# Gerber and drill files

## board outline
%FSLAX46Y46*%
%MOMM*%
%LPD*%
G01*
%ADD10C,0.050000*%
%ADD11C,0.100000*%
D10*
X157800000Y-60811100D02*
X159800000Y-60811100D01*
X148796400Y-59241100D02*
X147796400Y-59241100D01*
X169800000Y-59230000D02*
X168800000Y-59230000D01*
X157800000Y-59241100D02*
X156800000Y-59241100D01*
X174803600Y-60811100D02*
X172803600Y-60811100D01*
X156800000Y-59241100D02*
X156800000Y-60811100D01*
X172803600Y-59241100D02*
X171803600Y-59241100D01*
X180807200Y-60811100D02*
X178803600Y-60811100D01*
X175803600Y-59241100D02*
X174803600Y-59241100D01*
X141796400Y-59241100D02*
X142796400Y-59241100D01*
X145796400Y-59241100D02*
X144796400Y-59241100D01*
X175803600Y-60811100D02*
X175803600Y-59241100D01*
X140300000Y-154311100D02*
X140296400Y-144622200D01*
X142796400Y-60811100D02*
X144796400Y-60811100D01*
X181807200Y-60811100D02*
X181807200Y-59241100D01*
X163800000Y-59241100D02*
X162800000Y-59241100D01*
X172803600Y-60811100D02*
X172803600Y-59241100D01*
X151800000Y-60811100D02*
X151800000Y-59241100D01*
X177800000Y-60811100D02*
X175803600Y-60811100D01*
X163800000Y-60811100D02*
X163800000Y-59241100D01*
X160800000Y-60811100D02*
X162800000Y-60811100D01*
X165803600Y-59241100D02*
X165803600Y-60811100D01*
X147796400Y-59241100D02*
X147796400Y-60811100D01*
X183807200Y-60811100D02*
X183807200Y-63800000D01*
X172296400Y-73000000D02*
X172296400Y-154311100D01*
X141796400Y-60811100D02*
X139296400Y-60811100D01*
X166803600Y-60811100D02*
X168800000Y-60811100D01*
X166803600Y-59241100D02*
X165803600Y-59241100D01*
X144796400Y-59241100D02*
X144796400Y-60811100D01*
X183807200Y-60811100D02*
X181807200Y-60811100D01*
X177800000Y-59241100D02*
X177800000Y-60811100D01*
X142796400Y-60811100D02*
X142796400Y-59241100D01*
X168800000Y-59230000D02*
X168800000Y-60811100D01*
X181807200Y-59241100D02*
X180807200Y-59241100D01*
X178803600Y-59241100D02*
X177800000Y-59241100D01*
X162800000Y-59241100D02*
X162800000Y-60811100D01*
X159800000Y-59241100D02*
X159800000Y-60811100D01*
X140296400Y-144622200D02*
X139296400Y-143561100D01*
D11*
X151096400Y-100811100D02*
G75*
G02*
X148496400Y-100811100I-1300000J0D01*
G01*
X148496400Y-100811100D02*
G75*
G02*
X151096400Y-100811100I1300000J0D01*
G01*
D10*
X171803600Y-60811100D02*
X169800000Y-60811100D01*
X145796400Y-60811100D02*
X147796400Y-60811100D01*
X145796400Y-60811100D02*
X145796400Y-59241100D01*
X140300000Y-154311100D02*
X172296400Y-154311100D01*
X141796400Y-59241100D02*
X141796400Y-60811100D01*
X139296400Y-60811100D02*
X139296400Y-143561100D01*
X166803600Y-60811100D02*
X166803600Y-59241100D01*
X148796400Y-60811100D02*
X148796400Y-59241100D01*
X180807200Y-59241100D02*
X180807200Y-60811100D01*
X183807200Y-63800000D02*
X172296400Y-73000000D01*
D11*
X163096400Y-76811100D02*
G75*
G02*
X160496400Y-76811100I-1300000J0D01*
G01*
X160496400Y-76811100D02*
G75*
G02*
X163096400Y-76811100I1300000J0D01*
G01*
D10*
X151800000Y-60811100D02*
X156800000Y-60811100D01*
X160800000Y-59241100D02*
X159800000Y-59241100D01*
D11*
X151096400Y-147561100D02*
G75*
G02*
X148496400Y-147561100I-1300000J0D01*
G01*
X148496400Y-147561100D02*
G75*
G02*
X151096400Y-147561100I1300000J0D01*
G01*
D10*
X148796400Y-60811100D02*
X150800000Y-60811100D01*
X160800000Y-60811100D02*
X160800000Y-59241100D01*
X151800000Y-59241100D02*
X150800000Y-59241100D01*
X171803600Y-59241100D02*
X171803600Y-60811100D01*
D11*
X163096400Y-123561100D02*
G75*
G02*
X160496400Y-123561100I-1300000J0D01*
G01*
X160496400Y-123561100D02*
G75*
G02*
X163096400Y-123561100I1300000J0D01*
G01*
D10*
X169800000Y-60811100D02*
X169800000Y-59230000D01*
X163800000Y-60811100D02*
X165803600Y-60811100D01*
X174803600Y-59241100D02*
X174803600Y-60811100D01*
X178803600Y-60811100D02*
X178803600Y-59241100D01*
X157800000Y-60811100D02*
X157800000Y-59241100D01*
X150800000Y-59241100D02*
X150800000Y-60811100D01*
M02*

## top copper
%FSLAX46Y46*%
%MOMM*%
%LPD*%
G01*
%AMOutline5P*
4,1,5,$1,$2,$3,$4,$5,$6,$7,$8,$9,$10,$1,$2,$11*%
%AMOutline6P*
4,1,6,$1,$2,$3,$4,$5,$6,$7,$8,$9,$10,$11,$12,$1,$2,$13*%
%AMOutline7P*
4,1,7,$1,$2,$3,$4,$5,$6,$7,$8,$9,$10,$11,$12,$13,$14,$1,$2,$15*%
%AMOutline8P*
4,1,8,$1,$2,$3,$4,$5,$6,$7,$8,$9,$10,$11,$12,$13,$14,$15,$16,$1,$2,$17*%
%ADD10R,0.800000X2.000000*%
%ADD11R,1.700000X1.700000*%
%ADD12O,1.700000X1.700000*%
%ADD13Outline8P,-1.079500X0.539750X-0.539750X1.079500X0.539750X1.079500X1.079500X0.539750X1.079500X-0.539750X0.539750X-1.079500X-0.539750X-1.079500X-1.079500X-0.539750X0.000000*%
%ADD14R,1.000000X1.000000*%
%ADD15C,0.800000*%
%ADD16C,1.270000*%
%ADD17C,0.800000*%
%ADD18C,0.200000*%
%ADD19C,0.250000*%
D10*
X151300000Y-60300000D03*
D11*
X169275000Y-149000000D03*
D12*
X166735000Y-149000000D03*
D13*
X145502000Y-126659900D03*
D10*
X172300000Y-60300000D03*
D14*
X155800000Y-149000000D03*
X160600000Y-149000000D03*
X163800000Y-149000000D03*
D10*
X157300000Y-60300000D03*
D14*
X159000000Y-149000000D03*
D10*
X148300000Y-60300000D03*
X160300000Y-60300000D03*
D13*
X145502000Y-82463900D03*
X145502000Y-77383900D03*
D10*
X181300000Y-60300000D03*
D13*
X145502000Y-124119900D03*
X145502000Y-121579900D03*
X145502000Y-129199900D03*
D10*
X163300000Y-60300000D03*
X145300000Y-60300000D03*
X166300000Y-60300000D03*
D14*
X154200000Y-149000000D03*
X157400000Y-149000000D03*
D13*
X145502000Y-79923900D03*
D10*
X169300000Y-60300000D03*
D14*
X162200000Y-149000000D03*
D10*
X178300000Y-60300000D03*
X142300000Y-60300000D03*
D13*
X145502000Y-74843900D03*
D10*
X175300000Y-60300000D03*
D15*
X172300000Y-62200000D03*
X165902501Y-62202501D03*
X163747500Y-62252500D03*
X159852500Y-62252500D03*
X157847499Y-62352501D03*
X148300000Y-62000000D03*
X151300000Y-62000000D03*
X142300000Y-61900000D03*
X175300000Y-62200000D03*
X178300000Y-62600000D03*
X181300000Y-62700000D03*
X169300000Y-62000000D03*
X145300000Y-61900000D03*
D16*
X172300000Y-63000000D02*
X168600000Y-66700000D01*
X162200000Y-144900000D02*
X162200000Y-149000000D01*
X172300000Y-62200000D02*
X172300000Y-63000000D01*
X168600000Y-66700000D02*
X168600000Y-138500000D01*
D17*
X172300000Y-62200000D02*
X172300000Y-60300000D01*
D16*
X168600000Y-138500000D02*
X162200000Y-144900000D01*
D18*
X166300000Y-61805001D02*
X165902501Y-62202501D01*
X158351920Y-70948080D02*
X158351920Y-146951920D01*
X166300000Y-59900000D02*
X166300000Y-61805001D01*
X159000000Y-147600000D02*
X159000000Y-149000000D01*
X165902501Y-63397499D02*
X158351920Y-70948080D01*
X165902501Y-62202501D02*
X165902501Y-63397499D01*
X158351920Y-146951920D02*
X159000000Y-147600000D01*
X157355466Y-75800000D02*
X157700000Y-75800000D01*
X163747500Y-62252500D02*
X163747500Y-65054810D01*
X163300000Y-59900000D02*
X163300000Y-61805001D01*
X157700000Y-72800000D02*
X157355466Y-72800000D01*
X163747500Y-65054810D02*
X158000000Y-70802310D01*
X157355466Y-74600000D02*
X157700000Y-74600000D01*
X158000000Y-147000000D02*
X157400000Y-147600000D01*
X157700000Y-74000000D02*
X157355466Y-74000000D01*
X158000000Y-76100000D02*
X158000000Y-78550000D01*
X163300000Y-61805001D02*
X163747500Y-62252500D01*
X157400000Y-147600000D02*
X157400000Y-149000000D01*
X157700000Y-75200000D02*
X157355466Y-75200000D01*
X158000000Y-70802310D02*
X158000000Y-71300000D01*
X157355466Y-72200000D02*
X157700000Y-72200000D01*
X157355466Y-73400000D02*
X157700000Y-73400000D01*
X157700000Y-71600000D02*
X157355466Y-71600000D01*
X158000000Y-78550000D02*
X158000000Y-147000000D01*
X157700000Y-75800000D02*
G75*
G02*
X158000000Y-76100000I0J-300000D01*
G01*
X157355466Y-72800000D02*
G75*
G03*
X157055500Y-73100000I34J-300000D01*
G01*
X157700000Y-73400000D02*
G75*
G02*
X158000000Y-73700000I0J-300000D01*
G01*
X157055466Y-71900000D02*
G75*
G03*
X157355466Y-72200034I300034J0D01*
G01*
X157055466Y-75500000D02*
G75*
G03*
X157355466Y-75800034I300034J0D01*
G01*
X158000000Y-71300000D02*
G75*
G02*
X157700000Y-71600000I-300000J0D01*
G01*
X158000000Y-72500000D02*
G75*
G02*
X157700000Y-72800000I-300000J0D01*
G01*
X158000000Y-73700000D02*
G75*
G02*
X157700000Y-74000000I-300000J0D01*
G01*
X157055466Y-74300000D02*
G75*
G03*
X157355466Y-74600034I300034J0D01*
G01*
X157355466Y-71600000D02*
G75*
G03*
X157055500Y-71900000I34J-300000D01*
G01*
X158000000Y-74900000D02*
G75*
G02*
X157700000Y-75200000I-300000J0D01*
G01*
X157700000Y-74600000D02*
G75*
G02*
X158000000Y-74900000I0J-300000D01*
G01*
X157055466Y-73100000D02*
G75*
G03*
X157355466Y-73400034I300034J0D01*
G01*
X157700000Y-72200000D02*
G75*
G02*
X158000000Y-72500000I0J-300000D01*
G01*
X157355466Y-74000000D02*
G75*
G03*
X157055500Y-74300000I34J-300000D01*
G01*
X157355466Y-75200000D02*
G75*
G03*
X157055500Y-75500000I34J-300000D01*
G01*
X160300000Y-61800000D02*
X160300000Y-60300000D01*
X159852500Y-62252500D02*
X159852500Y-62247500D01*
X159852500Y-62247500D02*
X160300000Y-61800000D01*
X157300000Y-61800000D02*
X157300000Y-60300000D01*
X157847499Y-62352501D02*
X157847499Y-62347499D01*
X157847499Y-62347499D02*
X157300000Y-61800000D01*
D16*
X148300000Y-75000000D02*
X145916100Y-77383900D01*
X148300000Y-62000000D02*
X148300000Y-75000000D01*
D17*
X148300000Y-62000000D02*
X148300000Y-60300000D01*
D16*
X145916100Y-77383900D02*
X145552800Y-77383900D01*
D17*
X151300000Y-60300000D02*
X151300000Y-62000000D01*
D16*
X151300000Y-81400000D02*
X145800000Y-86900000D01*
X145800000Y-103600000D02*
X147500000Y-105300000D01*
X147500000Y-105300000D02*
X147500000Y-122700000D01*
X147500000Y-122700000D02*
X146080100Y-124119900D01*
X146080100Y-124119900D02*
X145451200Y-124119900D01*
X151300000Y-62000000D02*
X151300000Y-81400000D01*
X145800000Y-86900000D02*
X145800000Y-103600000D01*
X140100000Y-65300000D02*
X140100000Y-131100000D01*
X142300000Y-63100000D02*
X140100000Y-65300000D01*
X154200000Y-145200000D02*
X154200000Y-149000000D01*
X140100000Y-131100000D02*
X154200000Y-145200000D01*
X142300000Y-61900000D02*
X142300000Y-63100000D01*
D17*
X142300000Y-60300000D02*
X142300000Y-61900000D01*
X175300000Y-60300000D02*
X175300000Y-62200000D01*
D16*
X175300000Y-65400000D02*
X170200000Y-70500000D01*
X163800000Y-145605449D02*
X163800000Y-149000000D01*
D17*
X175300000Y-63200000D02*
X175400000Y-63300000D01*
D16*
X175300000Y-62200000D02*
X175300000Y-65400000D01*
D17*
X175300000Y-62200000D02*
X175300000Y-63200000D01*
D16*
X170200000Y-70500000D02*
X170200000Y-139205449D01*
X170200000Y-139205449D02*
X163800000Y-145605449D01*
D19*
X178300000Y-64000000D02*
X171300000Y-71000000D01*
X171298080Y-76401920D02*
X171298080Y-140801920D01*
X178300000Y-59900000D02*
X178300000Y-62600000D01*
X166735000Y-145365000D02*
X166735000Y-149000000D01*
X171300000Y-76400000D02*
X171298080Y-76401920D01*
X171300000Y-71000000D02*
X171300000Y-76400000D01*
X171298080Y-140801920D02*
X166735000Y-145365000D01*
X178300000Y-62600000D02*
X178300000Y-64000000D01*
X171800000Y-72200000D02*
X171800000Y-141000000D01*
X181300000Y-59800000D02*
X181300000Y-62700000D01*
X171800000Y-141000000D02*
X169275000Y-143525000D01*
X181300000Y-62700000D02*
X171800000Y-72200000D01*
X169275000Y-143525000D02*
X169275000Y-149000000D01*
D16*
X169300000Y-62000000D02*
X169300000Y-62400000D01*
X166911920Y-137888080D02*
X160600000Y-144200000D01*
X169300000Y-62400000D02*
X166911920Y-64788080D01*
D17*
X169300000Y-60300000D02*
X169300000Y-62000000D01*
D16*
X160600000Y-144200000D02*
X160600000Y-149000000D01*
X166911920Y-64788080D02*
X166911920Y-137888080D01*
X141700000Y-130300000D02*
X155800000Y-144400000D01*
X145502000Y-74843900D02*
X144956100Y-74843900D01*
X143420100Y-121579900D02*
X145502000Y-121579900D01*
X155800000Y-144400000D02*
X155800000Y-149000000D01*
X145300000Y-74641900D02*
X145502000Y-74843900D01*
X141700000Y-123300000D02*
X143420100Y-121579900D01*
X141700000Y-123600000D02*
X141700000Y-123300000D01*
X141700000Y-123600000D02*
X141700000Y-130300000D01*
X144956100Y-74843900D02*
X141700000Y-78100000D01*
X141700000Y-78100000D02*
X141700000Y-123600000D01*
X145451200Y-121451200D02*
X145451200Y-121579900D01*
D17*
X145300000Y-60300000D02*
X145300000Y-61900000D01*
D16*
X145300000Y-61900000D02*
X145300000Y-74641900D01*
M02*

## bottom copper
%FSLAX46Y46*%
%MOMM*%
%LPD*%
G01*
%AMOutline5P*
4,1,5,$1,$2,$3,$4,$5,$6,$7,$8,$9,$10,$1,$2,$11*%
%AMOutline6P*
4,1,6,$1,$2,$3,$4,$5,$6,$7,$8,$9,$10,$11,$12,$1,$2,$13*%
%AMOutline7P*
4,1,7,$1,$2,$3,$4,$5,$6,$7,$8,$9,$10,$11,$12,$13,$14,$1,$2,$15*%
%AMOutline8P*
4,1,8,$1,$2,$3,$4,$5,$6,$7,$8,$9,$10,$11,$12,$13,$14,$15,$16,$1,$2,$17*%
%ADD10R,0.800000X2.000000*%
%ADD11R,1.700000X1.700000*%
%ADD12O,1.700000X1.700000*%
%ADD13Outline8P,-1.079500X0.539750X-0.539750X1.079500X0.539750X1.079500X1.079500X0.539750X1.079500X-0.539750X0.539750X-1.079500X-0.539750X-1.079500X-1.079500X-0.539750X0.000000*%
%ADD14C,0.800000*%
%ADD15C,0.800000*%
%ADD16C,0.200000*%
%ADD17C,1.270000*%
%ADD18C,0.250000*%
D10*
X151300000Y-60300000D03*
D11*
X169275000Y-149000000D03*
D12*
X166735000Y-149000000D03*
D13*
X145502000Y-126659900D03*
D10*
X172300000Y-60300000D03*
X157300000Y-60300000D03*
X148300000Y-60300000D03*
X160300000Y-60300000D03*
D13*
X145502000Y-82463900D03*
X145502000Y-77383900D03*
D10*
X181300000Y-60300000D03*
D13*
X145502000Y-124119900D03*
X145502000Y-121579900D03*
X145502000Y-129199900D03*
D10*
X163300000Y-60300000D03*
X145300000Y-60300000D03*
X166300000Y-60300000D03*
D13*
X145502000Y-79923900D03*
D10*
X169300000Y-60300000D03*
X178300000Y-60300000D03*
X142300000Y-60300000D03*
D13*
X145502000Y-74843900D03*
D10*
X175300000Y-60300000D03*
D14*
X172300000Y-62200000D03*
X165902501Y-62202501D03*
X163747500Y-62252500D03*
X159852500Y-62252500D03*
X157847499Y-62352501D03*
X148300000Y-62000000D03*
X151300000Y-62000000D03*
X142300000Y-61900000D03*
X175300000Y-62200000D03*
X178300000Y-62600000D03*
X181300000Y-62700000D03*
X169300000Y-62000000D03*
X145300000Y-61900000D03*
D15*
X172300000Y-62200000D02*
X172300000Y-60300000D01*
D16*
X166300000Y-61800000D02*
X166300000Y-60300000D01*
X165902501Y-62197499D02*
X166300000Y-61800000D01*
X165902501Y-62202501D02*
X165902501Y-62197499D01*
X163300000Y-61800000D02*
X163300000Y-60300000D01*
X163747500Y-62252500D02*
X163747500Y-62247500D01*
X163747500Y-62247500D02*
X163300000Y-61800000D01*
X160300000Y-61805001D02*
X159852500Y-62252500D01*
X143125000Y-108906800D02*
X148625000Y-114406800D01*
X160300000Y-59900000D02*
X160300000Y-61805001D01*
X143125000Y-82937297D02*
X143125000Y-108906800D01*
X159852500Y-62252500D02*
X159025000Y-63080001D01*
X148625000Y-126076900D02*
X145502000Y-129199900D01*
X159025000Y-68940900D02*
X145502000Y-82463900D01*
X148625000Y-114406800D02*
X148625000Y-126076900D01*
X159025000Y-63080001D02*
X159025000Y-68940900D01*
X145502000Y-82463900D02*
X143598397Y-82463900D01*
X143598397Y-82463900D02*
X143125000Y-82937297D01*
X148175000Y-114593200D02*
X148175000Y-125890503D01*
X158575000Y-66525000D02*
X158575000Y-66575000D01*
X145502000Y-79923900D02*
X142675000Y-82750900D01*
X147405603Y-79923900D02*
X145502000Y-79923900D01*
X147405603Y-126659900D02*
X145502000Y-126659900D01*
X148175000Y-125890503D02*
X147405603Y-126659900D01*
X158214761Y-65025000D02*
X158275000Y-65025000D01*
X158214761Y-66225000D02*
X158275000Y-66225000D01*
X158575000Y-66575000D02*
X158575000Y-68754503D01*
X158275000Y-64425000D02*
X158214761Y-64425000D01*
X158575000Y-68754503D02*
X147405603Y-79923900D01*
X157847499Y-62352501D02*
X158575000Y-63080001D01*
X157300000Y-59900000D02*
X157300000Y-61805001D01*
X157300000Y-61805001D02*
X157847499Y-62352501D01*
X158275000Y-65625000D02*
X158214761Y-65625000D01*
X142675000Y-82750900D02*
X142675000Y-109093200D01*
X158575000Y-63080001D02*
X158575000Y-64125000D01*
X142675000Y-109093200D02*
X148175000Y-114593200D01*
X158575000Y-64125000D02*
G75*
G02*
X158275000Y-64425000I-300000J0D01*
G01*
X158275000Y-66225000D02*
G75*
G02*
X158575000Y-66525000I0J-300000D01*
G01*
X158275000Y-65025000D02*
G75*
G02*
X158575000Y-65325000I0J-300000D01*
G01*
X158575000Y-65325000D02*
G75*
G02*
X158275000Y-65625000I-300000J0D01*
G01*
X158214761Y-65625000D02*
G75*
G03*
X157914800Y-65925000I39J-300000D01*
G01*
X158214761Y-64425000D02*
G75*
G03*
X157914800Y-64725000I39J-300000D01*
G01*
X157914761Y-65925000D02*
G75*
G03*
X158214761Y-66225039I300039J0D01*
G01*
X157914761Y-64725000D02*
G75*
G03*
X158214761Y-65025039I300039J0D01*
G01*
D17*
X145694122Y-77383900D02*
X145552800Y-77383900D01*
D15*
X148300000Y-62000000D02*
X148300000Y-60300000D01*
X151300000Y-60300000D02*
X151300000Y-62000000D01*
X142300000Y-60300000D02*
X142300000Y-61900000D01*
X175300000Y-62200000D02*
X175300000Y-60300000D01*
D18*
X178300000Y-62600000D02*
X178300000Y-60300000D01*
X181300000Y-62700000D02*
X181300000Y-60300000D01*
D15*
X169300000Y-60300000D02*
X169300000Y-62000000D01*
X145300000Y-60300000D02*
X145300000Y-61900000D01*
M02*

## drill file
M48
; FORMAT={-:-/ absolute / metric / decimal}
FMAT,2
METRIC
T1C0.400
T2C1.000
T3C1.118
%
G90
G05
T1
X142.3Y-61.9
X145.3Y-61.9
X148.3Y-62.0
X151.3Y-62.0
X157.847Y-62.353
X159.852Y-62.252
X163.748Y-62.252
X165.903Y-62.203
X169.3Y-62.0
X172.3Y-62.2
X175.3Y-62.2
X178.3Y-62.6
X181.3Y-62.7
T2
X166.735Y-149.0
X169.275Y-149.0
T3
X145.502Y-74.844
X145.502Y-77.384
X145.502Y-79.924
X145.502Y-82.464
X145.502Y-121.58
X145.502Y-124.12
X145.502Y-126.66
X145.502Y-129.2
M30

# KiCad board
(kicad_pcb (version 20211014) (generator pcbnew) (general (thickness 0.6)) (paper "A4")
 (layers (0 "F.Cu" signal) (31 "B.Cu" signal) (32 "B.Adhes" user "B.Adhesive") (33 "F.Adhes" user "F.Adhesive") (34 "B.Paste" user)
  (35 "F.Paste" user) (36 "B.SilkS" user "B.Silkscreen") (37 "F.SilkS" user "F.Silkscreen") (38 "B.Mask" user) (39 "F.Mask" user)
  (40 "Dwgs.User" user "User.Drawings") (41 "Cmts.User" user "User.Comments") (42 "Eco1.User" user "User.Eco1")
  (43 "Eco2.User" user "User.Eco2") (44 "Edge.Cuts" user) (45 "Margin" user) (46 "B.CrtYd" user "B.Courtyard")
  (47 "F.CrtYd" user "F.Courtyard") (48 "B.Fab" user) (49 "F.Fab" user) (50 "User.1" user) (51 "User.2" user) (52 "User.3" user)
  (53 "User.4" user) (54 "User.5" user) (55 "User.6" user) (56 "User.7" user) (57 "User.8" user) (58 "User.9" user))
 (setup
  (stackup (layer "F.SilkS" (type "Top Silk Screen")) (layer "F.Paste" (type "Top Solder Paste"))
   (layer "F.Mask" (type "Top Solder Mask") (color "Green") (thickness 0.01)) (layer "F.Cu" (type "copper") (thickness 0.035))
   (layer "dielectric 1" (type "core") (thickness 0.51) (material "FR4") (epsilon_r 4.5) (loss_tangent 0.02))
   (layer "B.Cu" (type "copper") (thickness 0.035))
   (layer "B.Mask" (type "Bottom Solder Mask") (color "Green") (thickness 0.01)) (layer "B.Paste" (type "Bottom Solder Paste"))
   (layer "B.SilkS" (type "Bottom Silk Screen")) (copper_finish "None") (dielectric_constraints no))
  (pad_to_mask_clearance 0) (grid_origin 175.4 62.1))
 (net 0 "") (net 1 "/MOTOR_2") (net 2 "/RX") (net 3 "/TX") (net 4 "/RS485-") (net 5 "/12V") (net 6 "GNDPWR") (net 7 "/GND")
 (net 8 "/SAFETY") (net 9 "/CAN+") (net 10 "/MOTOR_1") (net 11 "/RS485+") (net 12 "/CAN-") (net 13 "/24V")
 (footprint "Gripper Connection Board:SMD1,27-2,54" (layer "F.Cu") (at 151.3 60.3)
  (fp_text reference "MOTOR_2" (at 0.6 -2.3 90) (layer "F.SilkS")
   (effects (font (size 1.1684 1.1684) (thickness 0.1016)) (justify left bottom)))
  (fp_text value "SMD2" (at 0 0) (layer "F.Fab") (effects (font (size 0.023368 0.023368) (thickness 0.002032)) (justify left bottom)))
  (pad "1" smd rect (at 0 0) (size 0.8 2) (layers "F.Cu" "F.Paste" "F.Mask") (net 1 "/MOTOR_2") (solder_mask_margin 0.1016))
  (pad "2" smd rect (at 0 0) (size 0.8 2) (layers "B.Cu" "B.Paste" "B.Mask") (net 1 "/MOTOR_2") (solder_mask_margin 0.1016)))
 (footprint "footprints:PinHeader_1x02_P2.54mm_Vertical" (layer "F.Cu") (at 169.275 149 -90)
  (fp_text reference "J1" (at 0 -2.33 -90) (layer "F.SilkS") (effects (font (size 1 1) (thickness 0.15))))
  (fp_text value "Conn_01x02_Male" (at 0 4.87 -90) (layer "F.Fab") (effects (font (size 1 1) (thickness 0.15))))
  (pad "1" thru_hole rect locked (at 0 0 270) (size 1.7 1.7) (drill 1) (layers *.Cu *.Mask) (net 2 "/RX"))
  (pad "2" thru_hole oval locked (at 0 2.54 270) (size 1.7 1.7) (drill 1) (layers *.Cu *.Mask) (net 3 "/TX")))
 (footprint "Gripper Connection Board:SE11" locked (layer "F.Cu") (at 145.502 126.6599)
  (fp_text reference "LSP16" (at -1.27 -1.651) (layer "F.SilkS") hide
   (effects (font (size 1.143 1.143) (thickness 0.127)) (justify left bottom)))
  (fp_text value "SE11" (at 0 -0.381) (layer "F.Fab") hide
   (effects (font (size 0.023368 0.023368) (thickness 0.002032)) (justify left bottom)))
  (pad "MP" thru_hole roundrect locked (at 0 0) (size 2.159 2.159) (drill 1.1176) (layers *.Cu *.Mask) (roundrect_rratio 0.25)
   (chamfer_ratio 0.25) (chamfer top_left top_right bottom_left bottom_right) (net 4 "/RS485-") (solder_mask_margin 0.1016)))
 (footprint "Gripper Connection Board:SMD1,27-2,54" (layer "F.Cu") (at 172.3 60.3)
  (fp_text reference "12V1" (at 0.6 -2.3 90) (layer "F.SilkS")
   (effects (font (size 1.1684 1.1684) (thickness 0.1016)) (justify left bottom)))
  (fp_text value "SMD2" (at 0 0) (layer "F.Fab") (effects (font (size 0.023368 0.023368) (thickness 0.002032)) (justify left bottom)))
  (pad "1" smd rect (at 0 0) (size 0.8 2) (layers "F.Cu" "F.Paste" "F.Mask") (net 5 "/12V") (solder_mask_margin 0.1016))
  (pad "2" smd rect (at 0 0) (size 0.8 2) (layers "B.Cu" "B.Paste" "B.Mask") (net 5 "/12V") (solder_mask_margin 0.1016)))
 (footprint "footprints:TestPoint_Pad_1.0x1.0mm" (layer "F.Cu") (at 155.8 149)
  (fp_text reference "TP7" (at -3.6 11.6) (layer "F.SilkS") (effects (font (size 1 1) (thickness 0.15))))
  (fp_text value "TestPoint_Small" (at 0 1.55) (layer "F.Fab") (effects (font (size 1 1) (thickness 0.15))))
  (pad "1" smd rect locked (at 0 0) (size 1 1) (layers "F.Cu" "F.Mask") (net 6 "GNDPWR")))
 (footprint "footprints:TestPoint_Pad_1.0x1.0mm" (layer "F.Cu") (at 160.6 149)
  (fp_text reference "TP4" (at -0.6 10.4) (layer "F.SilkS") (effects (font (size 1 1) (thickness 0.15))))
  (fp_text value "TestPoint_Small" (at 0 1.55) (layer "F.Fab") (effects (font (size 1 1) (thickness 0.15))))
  (pad "1" smd rect locked (at 0 0) (size 1 1) (layers "F.Cu" "F.Mask") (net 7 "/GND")))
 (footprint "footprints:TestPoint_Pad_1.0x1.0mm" (layer "F.Cu") (at 163.8 149)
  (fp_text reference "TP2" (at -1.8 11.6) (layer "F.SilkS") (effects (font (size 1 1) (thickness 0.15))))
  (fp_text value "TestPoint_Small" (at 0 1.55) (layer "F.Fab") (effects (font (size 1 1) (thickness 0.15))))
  (pad "1" smd rect locked (at 0 0) (size 1 1) (layers "F.Cu" "F.Mask") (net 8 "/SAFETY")))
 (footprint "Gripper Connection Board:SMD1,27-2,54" (layer "F.Cu") (at 157.3 60.3)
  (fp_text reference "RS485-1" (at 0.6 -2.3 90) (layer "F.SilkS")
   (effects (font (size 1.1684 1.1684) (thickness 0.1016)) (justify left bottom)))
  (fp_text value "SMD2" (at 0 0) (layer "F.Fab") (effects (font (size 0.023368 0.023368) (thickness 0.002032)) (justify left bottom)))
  (pad "1" smd rect (at 0 0) (size 0.8 2) (layers "F.Cu" "F.Paste" "F.Mask") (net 4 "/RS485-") (solder_mask_margin 0.1016))
  (pad "2" smd rect (at 0 0) (size 0.8 2) (layers "B.Cu" "B.Paste" "B.Mask") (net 4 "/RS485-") (solder_mask_margin 0.1016)))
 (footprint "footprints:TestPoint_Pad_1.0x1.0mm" (layer "F.Cu") (at 159 149)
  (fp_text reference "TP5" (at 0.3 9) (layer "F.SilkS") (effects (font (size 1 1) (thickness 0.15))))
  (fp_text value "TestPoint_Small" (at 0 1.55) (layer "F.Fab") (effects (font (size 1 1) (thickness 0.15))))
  (pad "1" smd rect locked (at 0 0) (size 1 1) (layers "F.Cu" "F.Mask") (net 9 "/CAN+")))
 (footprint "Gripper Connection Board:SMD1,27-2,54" (layer "F.Cu") (at 148.3 60.3)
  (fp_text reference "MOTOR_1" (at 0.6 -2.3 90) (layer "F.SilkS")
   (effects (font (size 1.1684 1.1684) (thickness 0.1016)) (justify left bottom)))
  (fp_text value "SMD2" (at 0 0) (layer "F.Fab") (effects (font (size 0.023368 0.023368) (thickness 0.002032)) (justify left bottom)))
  (pad "1" smd rect (at 0 0) (size 0.8 2) (layers "F.Cu" "F.Paste" "F.Mask") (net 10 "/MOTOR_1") (solder_mask_margin 0.1016))
  (pad "2" smd rect (at 0 0) (size 0.8 2) (layers "B.Cu" "B.Paste" "B.Mask") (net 10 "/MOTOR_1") (solder_mask_margin 0.1016)))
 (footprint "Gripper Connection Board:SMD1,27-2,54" (layer "F.Cu") (at 160.3 60.3)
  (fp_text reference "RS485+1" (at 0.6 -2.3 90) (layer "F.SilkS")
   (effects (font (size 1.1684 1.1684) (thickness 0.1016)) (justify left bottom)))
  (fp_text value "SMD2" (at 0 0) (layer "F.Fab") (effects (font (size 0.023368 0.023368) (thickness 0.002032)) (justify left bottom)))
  (pad "1" smd rect (at 0 0) (size 0.8 2) (layers "F.Cu" "F.Paste" "F.Mask") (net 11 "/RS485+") (solder_mask_margin 0.1016))
  (pad "2" smd rect (at 0 0) (size 0.8 2) (layers "B.Cu" "B.Paste" "B.Mask") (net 11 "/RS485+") (solder_mask_margin 0.1016)))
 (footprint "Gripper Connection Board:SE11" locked (layer "F.Cu") (at 145.502 82.4639)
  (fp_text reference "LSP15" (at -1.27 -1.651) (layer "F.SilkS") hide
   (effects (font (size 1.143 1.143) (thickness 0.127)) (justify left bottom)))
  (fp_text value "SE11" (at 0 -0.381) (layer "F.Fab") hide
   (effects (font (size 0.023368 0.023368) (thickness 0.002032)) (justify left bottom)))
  (pad "MP" thru_hole roundrect locked (at 0 0) (size 2.159 2.159) (drill 1.1176) (layers *.Cu *.Mask) (roundrect_rratio 0.25)
   (chamfer_ratio 0.25) (chamfer top_left top_right bottom_left bottom_right) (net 11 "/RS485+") (solder_mask_margin 0.1016)))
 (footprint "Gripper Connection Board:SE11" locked (layer "F.Cu") (at 145.502 77.3839)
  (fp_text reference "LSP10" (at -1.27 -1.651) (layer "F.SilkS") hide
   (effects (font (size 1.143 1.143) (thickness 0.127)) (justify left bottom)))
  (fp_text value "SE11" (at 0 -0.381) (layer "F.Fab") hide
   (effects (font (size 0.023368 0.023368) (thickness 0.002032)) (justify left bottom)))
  (pad "MP" thru_hole roundrect locked (at 0 0) (size 2.159 2.159) (drill 1.1176) (layers *.Cu *.Mask) (roundrect_rratio 0.25)
   (chamfer_ratio 0.25) (chamfer top_left top_right bottom_left bottom_right) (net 10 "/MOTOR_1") (solder_mask_margin 0.1016)))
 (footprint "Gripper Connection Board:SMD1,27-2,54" (layer "F.Cu") (at 181.3 60.3)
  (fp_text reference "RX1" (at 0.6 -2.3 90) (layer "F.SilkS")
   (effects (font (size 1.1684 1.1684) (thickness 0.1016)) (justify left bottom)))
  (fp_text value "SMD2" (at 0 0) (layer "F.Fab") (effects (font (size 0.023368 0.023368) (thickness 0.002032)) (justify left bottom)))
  (pad "1" smd rect (at 0 0) (size 0.8 2) (layers "F.Cu" "F.Paste" "F.Mask") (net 2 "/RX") (solder_mask_margin 0.1016))
  (pad "2" smd rect (at 0 0) (size 0.8 2) (layers "B.Cu" "B.Paste" "B.Mask") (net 2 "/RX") (solder_mask_margin 0.1016)))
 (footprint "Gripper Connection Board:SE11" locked (layer "F.Cu") (at 145.502 124.1199)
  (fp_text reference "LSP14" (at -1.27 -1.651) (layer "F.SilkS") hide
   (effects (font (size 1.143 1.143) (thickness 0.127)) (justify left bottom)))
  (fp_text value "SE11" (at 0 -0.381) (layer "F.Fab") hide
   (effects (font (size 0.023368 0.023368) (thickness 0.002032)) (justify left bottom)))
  (pad "MP" thru_hole roundrect locked (at 0 0) (size 2.159 2.159) (drill 1.1176) (layers *.Cu *.Mask) (roundrect_rratio 0.25)
   (chamfer_ratio 0.25) (chamfer top_left top_right bottom_left bottom_right) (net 1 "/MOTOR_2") (solder_mask_margin 0.1016)))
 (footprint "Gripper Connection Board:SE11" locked (layer "F.Cu") (at 145.502 121.5799)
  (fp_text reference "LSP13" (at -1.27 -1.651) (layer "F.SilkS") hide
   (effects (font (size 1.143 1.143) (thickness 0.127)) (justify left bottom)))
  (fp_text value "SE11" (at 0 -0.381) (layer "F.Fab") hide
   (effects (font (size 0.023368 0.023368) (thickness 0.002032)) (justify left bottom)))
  (pad "MP" thru_hole roundrect locked (at 0 0) (size 2.159 2.159) (drill 1.1176) (layers *.Cu *.Mask) (roundrect_rratio 0.25)
   (chamfer_ratio 0.25) (chamfer top_left top_right bottom_left bottom_right) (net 6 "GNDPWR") (solder_mask_margin 0.1016)))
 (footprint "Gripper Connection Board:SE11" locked (layer "F.Cu") (at 145.502 129.1999)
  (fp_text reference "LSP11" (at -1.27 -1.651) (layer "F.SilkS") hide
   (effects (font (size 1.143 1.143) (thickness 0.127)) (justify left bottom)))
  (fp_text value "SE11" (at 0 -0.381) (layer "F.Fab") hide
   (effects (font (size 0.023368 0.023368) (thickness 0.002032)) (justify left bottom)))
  (pad "MP" thru_hole roundrect locked (at 0 0) (size 2.159 2.159) (drill 1.1176) (layers *.Cu *.Mask) (roundrect_rratio 0.25)
   (chamfer_ratio 0.25) (chamfer top_left top_right bottom_left bottom_right) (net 11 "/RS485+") (solder_mask_margin 0.1016)))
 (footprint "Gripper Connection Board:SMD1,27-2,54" (layer "F.Cu") (at 163.3 60.3)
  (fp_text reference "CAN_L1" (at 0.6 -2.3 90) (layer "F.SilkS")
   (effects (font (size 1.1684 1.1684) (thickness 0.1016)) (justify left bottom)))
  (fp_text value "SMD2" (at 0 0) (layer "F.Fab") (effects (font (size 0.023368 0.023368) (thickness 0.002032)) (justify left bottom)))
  (pad "1" smd rect (at 0 0) (size 0.8 2) (layers "F.Cu" "F.Paste" "F.Mask") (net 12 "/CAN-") (solder_mask_margin 0.1016))
  (pad "2" smd rect (at 0 0) (size 0.8 2) (layers "B.Cu" "B.Paste" "B.Mask") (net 12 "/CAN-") (solder_mask_margin 0.1016)))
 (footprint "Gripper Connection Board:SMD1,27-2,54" (layer "F.Cu") (at 145.3 60.3)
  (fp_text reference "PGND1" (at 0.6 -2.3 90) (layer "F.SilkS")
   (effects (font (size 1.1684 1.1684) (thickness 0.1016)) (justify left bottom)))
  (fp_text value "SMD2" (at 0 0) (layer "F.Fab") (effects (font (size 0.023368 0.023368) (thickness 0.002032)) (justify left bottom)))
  (pad "1" smd rect (at 0 0) (size 0.8 2) (layers "F.Cu" "F.Paste" "F.Mask") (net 6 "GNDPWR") (solder_mask_margin 0.1016))
  (pad "2" smd rect (at 0 0) (size 0.8 2) (layers "B.Cu" "B.Paste" "B.Mask") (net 6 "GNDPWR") (solder_mask_margin 0.1016)))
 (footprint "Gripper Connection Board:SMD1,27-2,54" (layer "F.Cu") (at 166.3 60.3)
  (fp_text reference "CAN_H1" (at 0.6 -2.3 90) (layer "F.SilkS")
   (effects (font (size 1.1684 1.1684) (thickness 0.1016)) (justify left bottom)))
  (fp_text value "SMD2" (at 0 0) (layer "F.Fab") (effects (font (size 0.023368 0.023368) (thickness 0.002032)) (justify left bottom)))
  (pad "1" smd rect (at 0 0) (size 0.8 2) (layers "F.Cu" "F.Paste" "F.Mask") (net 9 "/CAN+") (solder_mask_margin 0.1016))
  (pad "2" smd rect (at 0 0) (size 0.8 2) (layers "B.Cu" "B.Paste" "B.Mask") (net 9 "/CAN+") (solder_mask_margin 0.1016)))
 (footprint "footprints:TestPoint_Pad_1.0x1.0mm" (layer "F.Cu") (at 154.2 149)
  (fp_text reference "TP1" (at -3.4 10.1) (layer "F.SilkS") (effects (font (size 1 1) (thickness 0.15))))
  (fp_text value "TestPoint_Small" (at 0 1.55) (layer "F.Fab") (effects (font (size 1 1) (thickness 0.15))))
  (pad "1" smd rect locked (at 0 0) (size 1 1) (layers "F.Cu" "F.Mask") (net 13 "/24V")))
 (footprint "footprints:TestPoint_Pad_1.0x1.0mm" (layer "F.Cu") (at 157.4 149)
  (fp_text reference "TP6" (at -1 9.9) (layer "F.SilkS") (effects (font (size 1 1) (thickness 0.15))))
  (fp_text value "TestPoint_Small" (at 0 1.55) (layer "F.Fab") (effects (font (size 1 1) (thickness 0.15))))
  (pad "1" smd rect locked (at 0 0) (size 1 1) (layers "F.Cu" "F.Mask") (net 12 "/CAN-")))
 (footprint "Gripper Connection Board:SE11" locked (layer "F.Cu") (at 145.502 79.9239)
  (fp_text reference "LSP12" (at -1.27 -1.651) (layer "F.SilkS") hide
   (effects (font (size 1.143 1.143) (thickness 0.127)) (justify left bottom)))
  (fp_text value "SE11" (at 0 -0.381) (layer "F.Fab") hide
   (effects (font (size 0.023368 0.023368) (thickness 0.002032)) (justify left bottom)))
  (pad "MP" thru_hole roundrect locked (at 0 0) (size 2.159 2.159) (drill 1.1176) (layers *.Cu *.Mask) (roundrect_rratio 0.25)
   (chamfer_ratio 0.25) (chamfer top_left top_right bottom_left bottom_right) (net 4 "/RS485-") (solder_mask_margin 0.1016)))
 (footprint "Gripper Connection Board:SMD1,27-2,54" (layer "F.Cu") (at 169.3 60.3)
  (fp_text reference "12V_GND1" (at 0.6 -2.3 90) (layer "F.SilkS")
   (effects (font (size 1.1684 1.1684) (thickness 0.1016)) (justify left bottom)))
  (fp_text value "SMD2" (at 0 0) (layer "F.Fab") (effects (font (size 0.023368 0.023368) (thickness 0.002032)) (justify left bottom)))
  (pad "1" smd rect (at 0 0) (size 0.8 2) (layers "F.Cu" "F.Paste" "F.Mask") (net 7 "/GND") (solder_mask_margin 0.1016))
  (pad "2" smd rect (at 0 0) (size 0.8 2) (layers "B.Cu" "B.Paste" "B.Mask") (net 7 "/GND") (solder_mask_margin 0.1016)))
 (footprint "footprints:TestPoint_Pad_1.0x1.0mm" (layer "F.Cu") (at 162.2 149)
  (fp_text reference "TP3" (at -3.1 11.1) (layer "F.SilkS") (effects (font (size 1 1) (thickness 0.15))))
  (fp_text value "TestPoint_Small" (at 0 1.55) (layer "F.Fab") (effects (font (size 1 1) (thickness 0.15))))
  (pad "1" smd rect locked (at 0 0) (size 1 1) (layers "F.Cu" "F.Mask") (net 5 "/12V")))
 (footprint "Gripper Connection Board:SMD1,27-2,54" (layer "F.Cu") (at 178.3 60.3)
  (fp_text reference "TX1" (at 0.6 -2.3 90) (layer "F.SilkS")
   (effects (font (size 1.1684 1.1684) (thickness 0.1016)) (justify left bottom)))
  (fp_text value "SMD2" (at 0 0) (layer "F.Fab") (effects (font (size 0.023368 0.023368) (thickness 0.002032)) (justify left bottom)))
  (pad "1" smd rect (at 0 0) (size 0.8 2) (layers "F.Cu" "F.Paste" "F.Mask") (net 3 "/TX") (solder_mask_margin 0.1016))
  (pad "2" smd rect (at 0 0) (size 0.8 2) (layers "B.Cu" "B.Paste" "B.Mask") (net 3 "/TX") (solder_mask_margin 0.1016)))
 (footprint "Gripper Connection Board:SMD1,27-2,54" (layer "F.Cu") (at 142.3 60.3)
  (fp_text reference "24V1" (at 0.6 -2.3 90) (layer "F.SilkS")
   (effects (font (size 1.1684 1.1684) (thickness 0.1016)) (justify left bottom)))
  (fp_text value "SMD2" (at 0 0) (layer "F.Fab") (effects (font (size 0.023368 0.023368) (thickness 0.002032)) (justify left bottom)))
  (pad "1" smd rect (at 0 0) (size 0.8 2) (layers "F.Cu" "F.Paste" "F.Mask") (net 13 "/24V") (solder_mask_margin 0.1016))
  (pad "2" smd rect (at 0 0) (size 0.8 2) (layers "B.Cu" "B.Paste" "B.Mask") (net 13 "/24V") (solder_mask_margin 0.1016)))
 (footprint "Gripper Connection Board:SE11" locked (layer "F.Cu") (at 145.502 74.8439)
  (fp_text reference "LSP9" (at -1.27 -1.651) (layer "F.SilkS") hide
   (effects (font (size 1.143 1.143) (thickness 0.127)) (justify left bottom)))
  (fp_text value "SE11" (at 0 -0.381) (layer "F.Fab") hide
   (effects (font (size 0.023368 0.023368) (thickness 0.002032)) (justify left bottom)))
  (pad "MP" thru_hole roundrect locked (at 0 0) (size 2.159 2.159) (drill 1.1176) (layers *.Cu *.Mask) (roundrect_rratio 0.25)
   (chamfer_ratio 0.25) (chamfer top_left top_right bottom_left bottom_right) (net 6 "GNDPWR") (solder_mask_margin 0.1016)))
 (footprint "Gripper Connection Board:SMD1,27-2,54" (layer "F.Cu") (at 175.3 60.3)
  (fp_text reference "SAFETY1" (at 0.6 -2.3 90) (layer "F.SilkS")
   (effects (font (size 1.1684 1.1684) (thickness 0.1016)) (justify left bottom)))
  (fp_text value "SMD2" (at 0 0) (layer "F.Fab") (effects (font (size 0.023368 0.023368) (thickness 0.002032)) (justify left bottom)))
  (pad "1" smd rect (at 0 0) (size 0.8 2) (layers "F.Cu" "F.Paste" "F.Mask") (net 8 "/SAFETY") (solder_mask_margin 0.1016))
  (pad "2" smd rect (at 0 0) (size 0.8 2) (layers "B.Cu" "B.Paste" "B.Mask") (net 8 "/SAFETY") (solder_mask_margin 0.1016)))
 (gr_line (start 157.8 60.8111) (end 159.8 60.8111) (layer "Edge.Cuts") (width 0.05))
 (gr_line (start 148.7964 59.2411) (end 147.7964 59.2411) (layer "Edge.Cuts") (width 0.05))
 (gr_line (start 169.8 59.23) (end 168.8 59.23) (layer "Edge.Cuts") (width 0.05))
 (gr_line (start 157.8 59.2411) (end 156.8 59.2411) (layer "Edge.Cuts") (width 0.05))
 (gr_line (start 174.8036 60.8111) (end 172.8036 60.8111) (layer "Edge.Cuts") (width 0.05))
 (gr_line (start 156.8 59.2411) (end 156.8 60.8111) (layer "Edge.Cuts") (width 0.05))
 (gr_line (start 172.8036 59.2411) (end 171.8036 59.2411) (layer "Edge.Cuts") (width 0.05))
 (gr_line (start 180.8072 60.8111) (end 178.8036 60.8111) (layer "Edge.Cuts") (width 0.05))
 (gr_line (start 175.8036 59.2411) (end 174.8036 59.2411) (layer "Edge.Cuts") (width 0.05))
 (gr_line (start 141.7964 59.2411) (end 142.7964 59.2411) (layer "Edge.Cuts") (width 0.05))
 (gr_line (start 145.7964 59.2411) (end 144.7964 59.2411) (layer "Edge.Cuts") (width 0.05))
 (gr_line (start 175.8036 60.8111) (end 175.8036 59.2411) (layer "Edge.Cuts") (width 0.05))
 (gr_line (start 140.3 154.3111) (end 140.2964 144.6222) (layer "Edge.Cuts") (width 0.05))
 (gr_line (start 142.7964 60.8111) (end 144.7964 60.8111) (layer "Edge.Cuts") (width 0.05))
 (gr_line (start 181.8072 60.8111) (end 181.8072 59.2411) (layer "Edge.Cuts") (width 0.05))
 (gr_line (start 163.8 59.2411) (end 162.8 59.2411) (layer "Edge.Cuts") (width 0.05))
 (gr_line (start 172.8036 60.8111) (end 172.8036 59.2411) (layer "Edge.Cuts") (width 0.05))
 (gr_line (start 151.8 60.8111) (end 151.8 59.2411) (layer "Edge.Cuts") (width 0.05))
 (gr_line (start 177.8 60.8111) (end 175.8036 60.8111) (layer "Edge.Cuts") (width 0.05))
 (gr_line (start 163.8 60.8111) (end 163.8 59.2411) (layer "Edge.Cuts") (width 0.05))
 (gr_line (start 160.8 60.8111) (end 162.8 60.8111) (layer "Edge.Cuts") (width 0.05))
 (gr_line (start 165.8036 59.2411) (end 165.8036 60.8111) (layer "Edge.Cuts") (width 0.05))
 (gr_line (start 147.7964 59.2411) (end 147.7964 60.8111) (layer "Edge.Cuts") (width 0.05))
 (gr_line (start 183.8072 60.8111) (end 183.8072 63.8) (layer "Edge.Cuts") (width 0.05))
 (gr_line (start 172.2964 73) (end 172.2964 154.3111) (layer "Edge.Cuts") (width 0.05))
 (gr_line (start 141.7964 60.8111) (end 139.2964 60.8111) (layer "Edge.Cuts") (width 0.05))
 (gr_line (start 166.8036 60.8111) (end 168.8 60.8111) (layer "Edge.Cuts") (width 0.05))
 (gr_line (start 166.8036 59.2411) (end 165.8036 59.2411) (layer "Edge.Cuts") (width 0.05))
 (gr_line (start 144.7964 59.2411) (end 144.7964 60.8111) (layer "Edge.Cuts") (width 0.05))
 (gr_line (start 183.8072 60.8111) (end 181.8072 60.8111) (layer "Edge.Cuts") (width 0.05))
 (gr_line (start 177.8 59.2411) (end 177.8 60.8111) (layer "Edge.Cuts") (width 0.05))
 (gr_line (start 142.7964 60.8111) (end 142.7964 59.2411) (layer "Edge.Cuts") (width 0.05))
 (gr_line (start 168.8 59.23) (end 168.8 60.8111) (layer "Edge.Cuts") (width 0.05))
 (gr_line (start 181.8072 59.2411) (end 180.8072 59.2411) (layer "Edge.Cuts") (width 0.05))
 (gr_line (start 178.8036 59.2411) (end 177.8 59.2411) (layer "Edge.Cuts") (width 0.05))
 (gr_line (start 162.8 59.2411) (end 162.8 60.8111) (layer "Edge.Cuts") (width 0.05))
 (gr_line (start 159.8 59.2411) (end 159.8 60.8111) (layer "Edge.Cuts") (width 0.05))
 (gr_line (start 140.2964 144.6222) (end 139.2964 143.5611) (layer "Edge.Cuts") (width 0.05))
 (gr_circle (center 149.7964 100.8111) (end 149.7964 102.1111) (layer "Edge.Cuts") (width 0.1) (fill none))
 (gr_line (start 171.8036 60.8111) (end 169.8 60.8111) (layer "Edge.Cuts") (width 0.05))
 (gr_line (start 145.7964 60.8111) (end 147.7964 60.8111) (layer "Edge.Cuts") (width 0.05))
 (gr_line (start 145.7964 60.8111) (end 145.7964 59.2411) (layer "Edge.Cuts") (width 0.05))
 (gr_line (start 140.3 154.3111) (end 172.2964 154.3111) (layer "Edge.Cuts") (width 0.05))
 (gr_line (start 141.7964 59.2411) (end 141.7964 60.8111) (layer "Edge.Cuts") (width 0.05))
 (gr_line (start 139.2964 60.8111) (end 139.2964 143.5611) (layer "Edge.Cuts") (width 0.05))
 (gr_line (start 166.8036 60.8111) (end 166.8036 59.2411) (layer "Edge.Cuts") (width 0.05))
 (gr_line (start 148.7964 60.8111) (end 148.7964 59.2411) (layer "Edge.Cuts") (width 0.05))
 (gr_line (start 180.8072 59.2411) (end 180.8072 60.8111) (layer "Edge.Cuts") (width 0.05))
 (gr_line (start 183.8072 63.8) (end 172.2964 73) (layer "Edge.Cuts") (width 0.05))
 (gr_circle (center 161.7964 76.8111) (end 161.7964 78.1111) (layer "Edge.Cuts") (width 0.1) (fill none))
 (gr_line (start 151.8 60.8111) (end 156.8 60.8111) (layer "Edge.Cuts") (width 0.05))
 (gr_line (start 160.8 59.2411) (end 159.8 59.2411) (layer "Edge.Cuts") (width 0.05))
 (gr_circle (center 149.7964 147.5611) (end 151.0964 147.5611) (layer "Edge.Cuts") (width 0.1) (fill none))
 (gr_line (start 148.7964 60.8111) (end 150.8 60.8111) (layer "Edge.Cuts") (width 0.05))
 (gr_line (start 160.8 60.8111) (end 160.8 59.2411) (layer "Edge.Cuts") (width 0.05))
 (gr_line (start 151.8 59.2411) (end 150.8 59.2411) (layer "Edge.Cuts") (width 0.05))
 (gr_line (start 171.8036 59.2411) (end 171.8036 60.8111) (layer "Edge.Cuts") (width 0.05))
 (gr_circle (center 161.7964 123.5611) (end 161.7964 124.8611) (layer "Edge.Cuts") (width 0.1) (fill none))
 (gr_line (start 169.8 60.8111) (end 169.8 59.23) (layer "Edge.Cuts") (width 0.05))
 (gr_line (start 163.8 60.8111) (end 165.8036 60.8111) (layer "Edge.Cuts") (width 0.05))
 (gr_line (start 174.8036 59.2411) (end 174.8036 60.8111) (layer "Edge.Cuts") (width 0.05))
 (gr_line (start 178.8036 60.8111) (end 178.8036 59.2411) (layer "Edge.Cuts") (width 0.05))
 (gr_line (start 157.8 60.8111) (end 157.8 59.2411) (layer "Edge.Cuts") (width 0.05))
 (gr_line (start 150.8 59.2411) (end 150.8 60.8111) (layer "Edge.Cuts") (width 0.05))
 (segment (start 172.3 63) (end 168.6 66.7) (width 1.27) (layer "F.Cu") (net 5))
 (segment (start 162.2 144.9) (end 162.2 149) (width 1.27) (layer "F.Cu") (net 5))
 (segment (start 172.3 62.2) (end 172.3 63) (width 1.27) (layer "F.Cu") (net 5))
 (segment (start 168.6 66.7) (end 168.6 138.5) (width 1.27) (layer "F.Cu") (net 5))
 (segment (start 172.3 62.2) (end 172.3 60.3) (width 0.8) (layer "F.Cu") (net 5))
 (segment (start 168.6 138.5) (end 162.2 144.9) (width 1.27) (layer "F.Cu") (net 5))
 (via (at 172.3 62.2) (size 0.8) (drill 0.4) (layers "F.Cu" "B.Cu") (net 5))
 (segment (start 172.3 62.2) (end 172.3 60.3) (width 0.8) (layer "B.Cu") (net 5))
 (segment (start 166.3 61.805001) (end 165.902501 62.202501) (width 0.2) (layer "F.Cu") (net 9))
 (segment (start 158.35192 70.94808) (end 158.35192 146.95192) (width 0.2) (layer "F.Cu") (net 9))
 (segment (start 166.3 59.9) (end 166.3 61.805001) (width 0.2) (layer "F.Cu") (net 9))
 (segment (start 159 147.6) (end 159 149) (width 0.2) (layer "F.Cu") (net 9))
 (segment (start 165.902501 63.397499) (end 158.35192 70.94808) (width 0.2) (layer "F.Cu") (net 9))
 (segment (start 165.902501 62.202501) (end 165.902501 63.397499) (width 0.2) (layer "F.Cu") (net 9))
 (segment (start 158.35192 146.95192) (end 159 147.6) (width 0.2) (layer "F.Cu") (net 9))
 (via (at 165.902501 62.202501) (size 0.8) (drill 0.4) (layers "F.Cu" "B.Cu") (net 9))
 (segment (start 166.3 61.8) (end 166.3 60.3) (width 0.2) (layer "B.Cu") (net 9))
 (segment (start 165.902501 62.197499) (end 166.3 61.8) (width 0.2) (layer "B.Cu") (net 9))
 (segment (start 165.902501 62.202501) (end 165.902501 62.197499) (width 0.2) (layer "B.Cu") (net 9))
 (segment (start 157.355466 75.8) (end 157.7 75.8) (width 0.2) (layer "F.Cu") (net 12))
 (segment (start 163.7475 62.2525) (end 163.7475 65.05481) (width 0.2) (layer "F.Cu") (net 12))
 (segment (start 163.3 59.9) (end 163.3 61.805001) (width 0.2) (layer "F.Cu") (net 12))
 (segment (start 157.7 72.8) (end 157.355466 72.8) (width 0.2) (layer "F.Cu") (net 12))
 (segment (start 163.7475 65.05481) (end 158 70.80231) (width 0.2) (layer "F.Cu") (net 12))
 (segment (start 157.355466 74.6) (end 157.7 74.6) (width 0.2) (layer "F.Cu") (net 12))
 (segment (start 158 147) (end 157.4 147.6) (width 0.2) (layer "F.Cu") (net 12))
 (segment (start 157.7 74) (end 157.355466 74) (width 0.2) (layer "F.Cu") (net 12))
 (segment (start 158 76.1) (end 158 78.55) (width 0.2) (layer "F.Cu") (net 12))
 (segment (start 163.3 61.805001) (end 163.7475 62.2525) (width 0.2) (layer "F.Cu") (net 12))
 (segment (start 157.4 147.6) (end 157.4 149) (width 0.2) (layer "F.Cu") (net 12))
 (segment (start 157.7 75.2) (end 157.355466 75.2) (width 0.2) (layer "F.Cu") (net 12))
 (segment (start 158 70.80231) (end 158 71.3) (width 0.2) (layer "F.Cu") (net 12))
 (segment (start 157.355466 72.2) (end 157.7 72.2) (width 0.2) (layer "F.Cu") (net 12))
 (segment (start 157.355466 73.4) (end 157.7 73.4) (width 0.2) (layer "F.Cu") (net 12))
 (segment (start 157.7 71.6) (end 157.355466 71.6) (width 0.2) (layer "F.Cu") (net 12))
 (segment (start 158 78.55) (end 158 147) (width 0.2) (layer "F.Cu") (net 12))
 (via (at 163.7475 62.2525) (size 0.8) (drill 0.4) (layers "F.Cu" "B.Cu") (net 12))
 (arc (start 157.7 75.8) (mid 157.912132 75.887868) (end 158 76.1) (width 0.2) (layer "F.Cu") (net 12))
 (arc (start 157.355466 72.8) (mid 157.143334 72.887868) (end 157.055466 73.1) (width 0.2) (layer "F.Cu") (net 12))
 (arc (start 157.7 73.4) (mid 157.912132 73.487868) (end 158 73.7) (width 0.2) (layer "F.Cu") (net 12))
 (arc (start 157.055466 71.9) (mid 157.143334 72.112132) (end 157.355466 72.2) (width 0.2) (layer "F.Cu") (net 12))
 (arc (start 157.055466 75.5) (mid 157.143334 75.712132) (end 157.355466 75.8) (width 0.2) (layer "F.Cu") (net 12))
 (arc (start 158 71.3) (mid 157.912132 71.512132) (end 157.7 71.6) (width 0.2) (layer "F.Cu") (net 12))
 (arc (start 158 72.5) (mid 157.912132 72.712132) (end 157.7 72.8) (width 0.2) (layer "F.Cu") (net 12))
 (arc (start 158 73.7) (mid 157.912132 73.912132) (end 157.7 74) (width 0.2) (layer "F.Cu") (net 12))
 (arc (start 157.055466 74.3) (mid 157.143334 74.512132) (end 157.355466 74.6) (width 0.2) (layer "F.Cu") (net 12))
 (arc (start 157.355466 71.6) (mid 157.143334 71.687868) (end 157.055466 71.9) (width 0.2) (layer "F.Cu") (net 12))
 (arc (start 158 74.9) (mid 157.912132 75.112132) (end 157.7 75.2) (width 0.2) (layer "F.Cu") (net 12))
 (arc (start 157.7 74.6) (mid 157.912132 74.687868) (end 158 74.9) (width 0.2) (layer "F.Cu") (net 12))
 (arc (start 157.055466 73.1) (mid 157.143334 73.312132) (end 157.355466 73.4) (width 0.2) (layer "F.Cu") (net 12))
 (arc (start 157.7 72.2) (mid 157.912132 72.287868) (end 158 72.5) (width 0.2) (layer "F.Cu") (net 12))
 (arc (start 157.355466 74) (mid 157.143334 74.087868) (end 157.055466 74.3) (width 0.2) (layer "F.Cu") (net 12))
 (arc (start 157.355466 75.2) (mid 157.143334 75.287868) (end 157.055466 75.5) (width 0.2) (layer "F.Cu") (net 12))
 (segment (start 163.3 61.8) (end 163.3 60.3) (width 0.2) (layer "B.Cu") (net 12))
 (segment (start 163.7475 62.2525) (end 163.7475 62.2475) (width 0.2) (layer "B.Cu") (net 12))
 (segment (start 163.7475 62.2475) (end 163.3 61.8) (width 0.2) (layer "B.Cu") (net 12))
 (segment (start 160.3 61.8) (end 160.3 60.3) (width 0.2) (layer "F.Cu") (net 11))
 (segment (start 159.8525 62.2525) (end 159.8525 62.2475) (width 0.2) (layer "F.Cu") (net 11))
 (segment (start 159.8525 62.2475) (end 160.3 61.8) (width 0.2) (layer "F.Cu") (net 11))
 (via (at 159.8525 62.2525) (size 0.8) (drill 0.4) (layers "F.Cu" "B.Cu") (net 11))
 (segment (start 160.3 61.805001) (end 159.8525 62.2525) (width 0.2) (layer "B.Cu") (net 11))
 (segment (start 143.125 108.9068) (end 148.625 114.4068) (width 0.2) (layer "B.Cu") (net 11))
 (segment (start 160.3 59.9) (end 160.3 61.805001) (width 0.2) (layer "B.Cu") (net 11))
 (segment (start 143.125 82.937297) (end 143.125 108.9068) (width 0.2) (layer "B.Cu") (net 11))
 (segment (start 159.8525 62.2525) (end 159.025 63.080001) (width 0.2) (layer "B.Cu") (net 11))
 (segment (start 148.625 126.0769) (end 145.502 129.1999) (width 0.2) (layer "B.Cu") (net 11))
 (segment (start 159.025 68.9409) (end 145.502 82.4639) (width 0.2) (layer "B.Cu") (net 11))
 (segment (start 148.625 114.4068) (end 148.625 126.0769) (width 0.2) (layer "B.Cu") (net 11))
 (segment (start 159.025 63.080001) (end 159.025 68.9409) (width 0.2) (layer "B.Cu") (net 11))
 (segment (start 145.502 82.4639) (end 143.598397 82.4639) (width 0.2) (layer "B.Cu") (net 11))
 (segment (start 143.598397 82.4639) (end 143.125 82.937297) (width 0.2) (layer "B.Cu") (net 11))
 (segment (start 157.3 61.8) (end 157.3 60.3) (width 0.2) (layer "F.Cu") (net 4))
 (segment (start 157.847499 62.352501) (end 157.847499 62.347499) (width 0.2) (layer "F.Cu") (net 4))
 (segment (start 157.847499 62.347499) (end 157.3 61.8) (width 0.2) (layer "F.Cu") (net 4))
 (via (at 157.847499 62.352501) (size 0.8) (drill 0.4) (layers "F.Cu" "B.Cu") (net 4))
 (segment (start 148.175 114.5932) (end 148.175 125.890503) (width 0.2) (layer "B.Cu") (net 4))
 (segment (start 158.575 66.525) (end 158.575 66.575) (width 0.2) (layer "B.Cu") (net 4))
 (segment (start 145.502 79.9239) (end 142.675 82.7509) (width 0.2) (layer "B.Cu") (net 4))
 (segment (start 147.405603 79.9239) (end 145.502 79.9239) (width 0.2) (layer "B.Cu") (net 4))
 (segment (start 147.405603 126.6599) (end 145.502 126.6599) (width 0.2) (layer "B.Cu") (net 4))
 (segment (start 148.175 125.890503) (end 147.405603 126.6599) (width 0.2) (layer "B.Cu") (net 4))
 (segment (start 158.214761 65.025) (end 158.275 65.025) (width 0.2) (layer "B.Cu") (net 4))
 (segment (start 158.214761 66.225) (end 158.275 66.225) (width 0.2) (layer "B.Cu") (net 4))
 (segment (start 158.575 66.575) (end 158.575 68.754503) (width 0.2) (layer "B.Cu") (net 4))
 (segment (start 158.275 64.425) (end 158.214761 64.425) (width 0.2) (layer "B.Cu") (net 4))
 (segment (start 158.575 68.754503) (end 147.405603 79.9239) (width 0.2) (layer "B.Cu") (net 4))
 (segment (start 157.847499 62.352501) (end 158.575 63.080001) (width 0.2) (layer "B.Cu") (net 4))
 (segment (start 157.3 59.9) (end 157.3 61.805001) (width 0.2) (layer "B.Cu") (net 4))
 (segment (start 157.3 61.805001) (end 157.847499 62.352501) (width 0.2) (layer "B.Cu") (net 4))
 (segment (start 158.275 65.625) (end 158.214761 65.625) (width 0.2) (layer "B.Cu") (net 4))
 (segment (start 142.675 82.7509) (end 142.675 109.0932) (width 0.2) (layer "B.Cu") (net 4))
 (segment (start 158.575 63.080001) (end 158.575 64.125) (width 0.2) (layer "B.Cu") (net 4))
 (segment (start 142.675 109.0932) (end 148.175 114.5932) (width 0.2) (layer "B.Cu") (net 4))
 (arc (start 158.575 64.125) (mid 158.487132 64.337132) (end 158.275 64.425) (width 0.2) (layer "B.Cu") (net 4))
 (arc (start 158.275 66.225) (mid 158.487132 66.312868) (end 158.575 66.525) (width 0.2) (layer "B.Cu") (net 4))
 (arc (start 158.275 65.025) (mid 158.487132 65.112868) (end 158.575 65.325) (width 0.2) (layer "B.Cu") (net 4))
 (arc (start 158.575 65.325) (mid 158.487132 65.537132) (end 158.275 65.625) (width 0.2) (layer "B.Cu") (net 4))
 (arc (start 158.214761 65.625) (mid 158.002629 65.712868) (end 157.914761 65.925) (width 0.2) (layer "B.Cu") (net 4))
 (arc (start 158.214761 64.425) (mid 158.002629 64.512868) (end 157.914761 64.725) (width 0.2) (layer "B.Cu") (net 4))
 (arc (start 157.914761 65.925) (mid 158.002629 66.137132) (end 158.214761 66.225) (width 0.2) (layer "B.Cu") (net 4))
 (arc (start 157.914761 64.725) (mid 158.002629 64.937132) (end 158.214761 65.025) (width 0.2) (layer "B.Cu") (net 4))
 (segment (start 148.3 75) (end 145.9161 77.3839) (width 1.27) (layer "F.Cu") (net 10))
 (segment (start 148.3 62) (end 148.3 75) (width 1.27) (layer "F.Cu") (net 10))
 (segment (start 148.3 62) (end 148.3 60.3) (width 0.8) (layer "F.Cu") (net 10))
 (segment (start 145.9161 77.3839) (end 145.5528 77.3839) (width 1.27) (layer "F.Cu") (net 10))
 (via (at 148.3 62) (size 0.8) (drill 0.4) (layers "F.Cu" "B.Cu") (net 10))
 (segment (start 145.694122 77.3839) (end 145.5528 77.3839) (width 1.27) (layer "B.Cu") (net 10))
 (segment (start 148.3 62) (end 148.3 60.3) (width 0.8) (layer "B.Cu") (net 10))
 (segment (start 151.3 60.3) (end 151.3 62) (width 0.8) (layer "F.Cu") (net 1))
 (segment (start 151.3 81.4) (end 145.8 86.9) (width 1.27) (layer "F.Cu") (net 1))
 (segment (start 145.8 103.6) (end 147.5 105.3) (width 1.27) (layer "F.Cu") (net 1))
 (segment (start 147.5 105.3) (end 147.5 122.7) (width 1.27) (layer "F.Cu") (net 1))
 (segment (start 147.5 122.7) (end 146.0801 124.1199) (width 1.27) (layer "F.Cu") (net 1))
 (segment (start 146.0801 124.1199) (end 145.4512 124.1199) (width 1.27) (layer "F.Cu") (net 1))
 (segment (start 151.3 62) (end 151.3 81.4) (width 1.27) (layer "F.Cu") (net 1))
 (segment (start 145.8 86.9) (end 145.8 103.6) (width 1.27) (layer "F.Cu") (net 1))
 (via (at 151.3 62) (size 0.8) (drill 0.4) (layers "F.Cu" "B.Cu") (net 1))
 (segment (start 151.3 60.3) (end 151.3 62) (width 0.8) (layer "B.Cu") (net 1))
 (segment (start 140.1 65.3) (end 140.1 131.1) (width 1.27) (layer "F.Cu") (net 13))
 (segment (start 142.3 63.1) (end 140.1 65.3) (width 1.27) (layer "F.Cu") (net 13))
 (segment (start 154.2 145.2) (end 154.2 149) (width 1.27) (layer "F.Cu") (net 13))
 (segment (start 140.1 131.1) (end 154.2 145.2) (width 1.27) (layer "F.Cu") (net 13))
 (segment (start 142.3 61.9) (end 142.3 63.1) (width 1.27) (layer "F.Cu") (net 13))
 (segment (start 142.3 60.3) (end 142.3 61.9) (width 0.8) (layer "F.Cu") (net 13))
 (via (at 142.3 61.9) (size 0.8) (drill 0.4) (layers "F.Cu" "B.Cu") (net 13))
 (segment (start 142.3 60.3) (end 142.3 61.9) (width 0.8) (layer "B.Cu") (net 13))
 (segment (start 175.3 60.3) (end 175.3 62.2) (width 0.8) (layer "F.Cu") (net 8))
 (segment (start 175.3 65.4) (end 170.2 70.5) (width 1.27) (layer "F.Cu") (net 8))
 (segment (start 163.8 145.605449) (end 163.8 149) (width 1.27) (layer "F.Cu") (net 8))
 (segment (start 175.3 63.2) (end 175.4 63.3) (width 0.8) (layer "F.Cu") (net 8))
 (segment (start 175.3 62.2) (end 175.3 65.4) (width 1.27) (layer "F.Cu") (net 8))
 (segment (start 175.3 62.2) (end 175.3 63.2) (width 0.8) (layer "F.Cu") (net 8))
 (segment (start 170.2 70.5) (end 170.2 139.205449) (width 1.27) (layer "F.Cu") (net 8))
 (segment (start 170.2 139.205449) (end 163.8 145.605449) (width 1.27) (layer "F.Cu") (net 8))
 (via (at 175.3 62.2) (size 0.8) (drill 0.4) (layers "F.Cu" "B.Cu") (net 8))
 (segment (start 175.3 62.2) (end 175.3 60.3) (width 0.8) (layer "B.Cu") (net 8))
 (segment (start 178.3 64) (end 171.3 71) (width 0.25) (layer "F.Cu") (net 3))
 (segment (start 171.29808 76.40192) (end 171.29808 140.80192) (width 0.25) (layer "F.Cu") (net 3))
 (segment (start 178.3 59.9) (end 178.3 62.6) (width 0.25) (layer "F.Cu") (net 3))
 (segment (start 166.735 145.365) (end 166.735 149) (width 0.25) (layer "F.Cu") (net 3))
 (segment (start 171.3 76.4) (end 171.29808 76.40192) (width 0.25) (layer "F.Cu") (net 3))
 (segment (start 171.3 71) (end 171.3 76.4) (width 0.25) (layer "F.Cu") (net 3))
 (segment (start 171.29808 140.80192) (end 166.735 145.365) (width 0.25) (layer "F.Cu") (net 3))
 (segment (start 178.3 62.6) (end 178.3 64) (width 0.25) (layer "F.Cu") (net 3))
 (via (at 178.3 62.6) (size 0.8) (drill 0.4) (layers "F.Cu" "B.Cu") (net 3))
 (segment (start 178.3 62.6) (end 178.3 60.3) (width 0.25) (layer "B.Cu") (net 3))
 (segment (start 171.8 72.2) (end 171.8 141) (width 0.25) (layer "F.Cu") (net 2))
 (segment (start 181.3 59.8) (end 181.3 62.7) (width 0.25) (layer "F.Cu") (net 2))
 (segment (start 171.8 141) (end 169.275 143.525) (width 0.25) (layer "F.Cu") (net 2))
 (segment (start 181.3 62.7) (end 171.8 72.2) (width 0.25) (layer "F.Cu") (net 2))
 (segment (start 169.275 143.525) (end 169.275 149) (width 0.25) (layer "F.Cu") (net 2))
 (via (at 181.3 62.7) (size 0.8) (drill 0.4) (layers "F.Cu" "B.Cu") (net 2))
 (segment (start 181.3 62.7) (end 181.3 60.3) (width 0.25) (layer "B.Cu") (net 2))
 (segment (start 169.3 62) (end 169.3 62.4) (width 1.27) (layer "F.Cu") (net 7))
 (segment (start 166.91192 137.88808) (end 160.6 144.2) (width 1.27) (layer "F.Cu") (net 7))
 (segment (start 169.3 62.4) (end 166.91192 64.78808) (width 1.27) (layer "F.Cu") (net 7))
 (segment (start 169.3 60.3) (end 169.3 62) (width 0.8) (layer "F.Cu") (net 7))
 (segment (start 160.6 144.2) (end 160.6 149) (width 1.27) (layer "F.Cu") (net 7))
 (segment (start 166.91192 64.78808) (end 166.91192 137.88808) (width 1.27) (layer "F.Cu") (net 7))
 (via (at 169.3 62) (size 0.8) (drill 0.4) (layers "F.Cu" "B.Cu") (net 7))
 (segment (start 169.3 60.3) (end 169.3 62) (width 0.8) (layer "B.Cu") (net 7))
 (segment (start 141.7 130.3) (end 155.8 144.4) (width 1.27) (layer "F.Cu") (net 6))
 (segment (start 145.502 74.8439) (end 144.9561 74.8439) (width 1.27) (layer "F.Cu") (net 6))
 (segment (start 143.4201 121.5799) (end 145.502 121.5799) (width 1.27) (layer "F.Cu") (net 6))
 (segment (start 155.8 144.4) (end 155.8 149) (width 1.27) (layer "F.Cu") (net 6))
 (segment (start 145.3 74.6419) (end 145.502 74.8439) (width 1.27) (layer "F.Cu") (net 6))
 (segment (start 141.7 123.3) (end 143.4201 121.5799) (width 1.27) (layer "F.Cu") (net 6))
 (segment (start 141.7 123.6) (end 141.7 123.3) (width 1.27) (layer "F.Cu") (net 6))
 (segment (start 141.7 123.6) (end 141.7 130.3) (width 1.27) (layer "F.Cu") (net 6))
 (segment (start 144.9561 74.8439) (end 141.7 78.1) (width 1.27) (layer "F.Cu") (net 6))
 (segment (start 141.7 78.1) (end 141.7 123.6) (width 1.27) (layer "F.Cu") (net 6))
 (segment (start 145.4512 121.4512) (end 145.4512 121.5799) (width 1.27) (layer "F.Cu") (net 6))
 (segment (start 145.3 60.3) (end 145.3 61.9) (width 0.8) (layer "F.Cu") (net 6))
 (segment (start 145.3 61.9) (end 145.3 74.6419) (width 1.27) (layer "F.Cu") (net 6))
 (via (at 145.3 61.9) (size 0.8) (drill 0.4) (layers "F.Cu" "B.Cu") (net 6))
 (segment (start 145.3 60.3) (end 145.3 61.9) (width 0.8) (layer "B.Cu") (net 6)))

